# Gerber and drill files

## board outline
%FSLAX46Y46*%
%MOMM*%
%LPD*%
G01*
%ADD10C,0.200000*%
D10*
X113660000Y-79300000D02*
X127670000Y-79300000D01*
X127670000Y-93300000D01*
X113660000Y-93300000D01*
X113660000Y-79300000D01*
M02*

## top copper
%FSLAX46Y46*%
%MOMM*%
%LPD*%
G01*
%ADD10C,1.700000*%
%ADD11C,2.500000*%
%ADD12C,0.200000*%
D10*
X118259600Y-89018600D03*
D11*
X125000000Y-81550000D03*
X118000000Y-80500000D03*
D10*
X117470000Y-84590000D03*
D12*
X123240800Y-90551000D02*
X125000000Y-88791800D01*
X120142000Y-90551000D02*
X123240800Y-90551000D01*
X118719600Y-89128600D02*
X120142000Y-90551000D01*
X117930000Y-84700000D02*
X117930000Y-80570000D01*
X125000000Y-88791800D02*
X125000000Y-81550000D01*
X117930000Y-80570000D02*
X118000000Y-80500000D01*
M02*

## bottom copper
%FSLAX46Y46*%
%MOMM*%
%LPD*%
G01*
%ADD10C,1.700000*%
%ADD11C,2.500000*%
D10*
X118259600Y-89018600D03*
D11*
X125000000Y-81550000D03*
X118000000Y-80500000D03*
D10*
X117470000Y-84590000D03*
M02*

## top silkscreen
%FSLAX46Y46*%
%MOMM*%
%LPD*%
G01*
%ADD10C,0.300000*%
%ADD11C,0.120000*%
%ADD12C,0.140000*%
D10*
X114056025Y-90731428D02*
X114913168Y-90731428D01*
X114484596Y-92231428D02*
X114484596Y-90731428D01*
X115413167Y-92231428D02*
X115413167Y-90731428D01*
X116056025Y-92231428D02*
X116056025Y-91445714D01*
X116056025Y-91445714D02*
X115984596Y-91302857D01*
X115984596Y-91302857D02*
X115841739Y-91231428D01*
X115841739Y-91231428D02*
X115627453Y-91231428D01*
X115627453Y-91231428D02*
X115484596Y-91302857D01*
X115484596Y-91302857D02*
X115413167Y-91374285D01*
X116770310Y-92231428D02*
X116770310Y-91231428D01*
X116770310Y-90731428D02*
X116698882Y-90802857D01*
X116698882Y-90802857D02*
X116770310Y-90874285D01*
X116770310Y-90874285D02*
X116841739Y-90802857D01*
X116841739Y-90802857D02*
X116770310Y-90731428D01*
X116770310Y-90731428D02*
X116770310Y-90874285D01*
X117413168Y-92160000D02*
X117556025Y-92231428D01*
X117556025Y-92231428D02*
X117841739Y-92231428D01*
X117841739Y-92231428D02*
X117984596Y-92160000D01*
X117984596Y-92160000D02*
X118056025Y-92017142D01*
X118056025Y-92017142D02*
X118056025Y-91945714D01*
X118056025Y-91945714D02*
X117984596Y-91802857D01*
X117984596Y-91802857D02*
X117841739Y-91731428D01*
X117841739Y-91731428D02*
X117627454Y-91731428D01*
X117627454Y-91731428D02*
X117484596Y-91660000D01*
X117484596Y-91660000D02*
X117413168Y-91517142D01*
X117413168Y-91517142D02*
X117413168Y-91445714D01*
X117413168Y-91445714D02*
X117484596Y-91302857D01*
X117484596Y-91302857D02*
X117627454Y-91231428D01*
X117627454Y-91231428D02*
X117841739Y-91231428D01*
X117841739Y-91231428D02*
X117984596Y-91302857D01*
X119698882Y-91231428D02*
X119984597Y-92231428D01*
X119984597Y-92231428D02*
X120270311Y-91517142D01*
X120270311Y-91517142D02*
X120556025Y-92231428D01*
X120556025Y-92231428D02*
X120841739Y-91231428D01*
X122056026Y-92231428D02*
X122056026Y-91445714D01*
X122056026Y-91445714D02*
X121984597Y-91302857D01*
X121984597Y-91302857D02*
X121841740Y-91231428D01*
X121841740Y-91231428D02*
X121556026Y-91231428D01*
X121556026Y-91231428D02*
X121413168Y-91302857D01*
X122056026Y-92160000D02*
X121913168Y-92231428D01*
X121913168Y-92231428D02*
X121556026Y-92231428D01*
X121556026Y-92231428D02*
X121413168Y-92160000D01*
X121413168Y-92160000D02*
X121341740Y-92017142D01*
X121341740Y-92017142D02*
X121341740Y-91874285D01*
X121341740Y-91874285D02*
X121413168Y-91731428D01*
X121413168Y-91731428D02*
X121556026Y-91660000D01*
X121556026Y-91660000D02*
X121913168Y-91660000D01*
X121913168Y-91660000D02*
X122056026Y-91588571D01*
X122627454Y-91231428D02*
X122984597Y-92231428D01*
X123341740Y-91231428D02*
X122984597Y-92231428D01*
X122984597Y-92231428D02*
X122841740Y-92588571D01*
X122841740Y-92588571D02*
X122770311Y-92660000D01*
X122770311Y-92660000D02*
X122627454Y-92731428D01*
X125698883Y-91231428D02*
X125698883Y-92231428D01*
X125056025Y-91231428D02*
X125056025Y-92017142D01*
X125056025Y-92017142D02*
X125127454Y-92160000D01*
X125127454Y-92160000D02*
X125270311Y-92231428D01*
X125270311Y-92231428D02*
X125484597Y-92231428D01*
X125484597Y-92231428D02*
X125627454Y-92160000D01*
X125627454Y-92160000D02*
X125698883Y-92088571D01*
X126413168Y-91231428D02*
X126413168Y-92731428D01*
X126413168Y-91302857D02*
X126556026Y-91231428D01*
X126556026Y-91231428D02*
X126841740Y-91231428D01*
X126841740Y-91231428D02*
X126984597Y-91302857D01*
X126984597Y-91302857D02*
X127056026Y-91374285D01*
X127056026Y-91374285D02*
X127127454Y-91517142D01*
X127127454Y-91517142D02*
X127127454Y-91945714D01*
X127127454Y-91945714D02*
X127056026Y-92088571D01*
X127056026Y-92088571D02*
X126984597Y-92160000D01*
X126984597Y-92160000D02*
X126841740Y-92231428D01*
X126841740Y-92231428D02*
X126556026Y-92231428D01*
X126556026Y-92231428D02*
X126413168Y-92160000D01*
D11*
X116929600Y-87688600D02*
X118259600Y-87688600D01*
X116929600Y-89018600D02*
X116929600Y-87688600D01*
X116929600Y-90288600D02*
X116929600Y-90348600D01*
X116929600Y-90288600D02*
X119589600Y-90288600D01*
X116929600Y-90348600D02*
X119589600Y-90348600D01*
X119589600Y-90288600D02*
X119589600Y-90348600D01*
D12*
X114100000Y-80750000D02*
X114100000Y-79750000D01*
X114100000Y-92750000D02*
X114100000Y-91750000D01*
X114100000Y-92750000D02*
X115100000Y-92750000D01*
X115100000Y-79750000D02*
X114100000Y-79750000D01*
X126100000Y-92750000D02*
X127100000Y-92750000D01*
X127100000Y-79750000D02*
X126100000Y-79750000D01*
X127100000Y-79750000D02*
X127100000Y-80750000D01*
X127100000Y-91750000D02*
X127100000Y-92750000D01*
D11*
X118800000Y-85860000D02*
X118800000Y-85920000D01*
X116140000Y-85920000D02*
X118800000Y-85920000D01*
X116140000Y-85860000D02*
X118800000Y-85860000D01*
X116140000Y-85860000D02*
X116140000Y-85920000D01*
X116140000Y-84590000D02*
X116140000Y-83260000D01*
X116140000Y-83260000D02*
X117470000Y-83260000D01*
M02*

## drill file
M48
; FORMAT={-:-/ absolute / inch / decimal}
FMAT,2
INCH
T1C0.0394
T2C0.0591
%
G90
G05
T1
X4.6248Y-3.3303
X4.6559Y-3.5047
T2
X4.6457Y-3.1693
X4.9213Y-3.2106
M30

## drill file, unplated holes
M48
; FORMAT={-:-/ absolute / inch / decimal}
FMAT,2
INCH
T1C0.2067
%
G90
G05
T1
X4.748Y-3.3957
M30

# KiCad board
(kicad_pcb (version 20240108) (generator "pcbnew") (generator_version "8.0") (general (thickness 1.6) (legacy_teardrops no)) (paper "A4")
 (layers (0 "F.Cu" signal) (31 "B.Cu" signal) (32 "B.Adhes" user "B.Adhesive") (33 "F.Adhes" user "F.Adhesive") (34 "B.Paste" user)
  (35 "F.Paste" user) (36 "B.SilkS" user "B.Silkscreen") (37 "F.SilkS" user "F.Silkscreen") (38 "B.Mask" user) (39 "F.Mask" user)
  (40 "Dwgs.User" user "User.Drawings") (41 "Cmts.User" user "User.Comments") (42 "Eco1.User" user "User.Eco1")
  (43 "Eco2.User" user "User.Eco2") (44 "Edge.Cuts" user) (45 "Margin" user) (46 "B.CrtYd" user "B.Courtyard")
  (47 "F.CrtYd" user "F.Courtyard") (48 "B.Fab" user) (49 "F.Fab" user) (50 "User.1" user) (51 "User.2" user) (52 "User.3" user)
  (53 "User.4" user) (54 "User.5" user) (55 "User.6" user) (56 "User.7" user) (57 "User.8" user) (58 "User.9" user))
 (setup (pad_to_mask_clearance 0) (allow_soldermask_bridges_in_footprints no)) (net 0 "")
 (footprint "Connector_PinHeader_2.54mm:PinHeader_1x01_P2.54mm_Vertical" (layer "F.Cu") (at 118.2596 89.0186)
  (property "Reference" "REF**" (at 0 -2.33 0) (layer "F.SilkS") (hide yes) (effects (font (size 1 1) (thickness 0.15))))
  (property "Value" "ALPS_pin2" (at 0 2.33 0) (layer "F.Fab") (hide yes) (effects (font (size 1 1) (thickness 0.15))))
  (fp_line (start -1.33 -1.33) (end 0 -1.33) (stroke (width 0.12) (type solid)) (layer "F.SilkS"))
  (fp_line (start -1.33 0) (end -1.33 -1.33) (stroke (width 0.12) (type solid)) (layer "F.SilkS"))
  (fp_line (start -1.33 1.27) (end -1.33 1.33) (stroke (width 0.12) (type solid)) (layer "F.SilkS"))
  (fp_line (start -1.33 1.27) (end 1.33 1.27) (stroke (width 0.12) (type solid)) (layer "F.SilkS"))
  (fp_line (start -1.33 1.33) (end 1.33 1.33) (stroke (width 0.12) (type solid)) (layer "F.SilkS"))
  (fp_line (start 1.33 1.27) (end 1.33 1.33) (stroke (width 0.12) (type solid)) (layer "F.SilkS"))
  (pad "2" thru_hole circle (at 0 0) (size 1.7 1.7) (drill 1) (layers "*.Cu" "*.Mask") (remove_unused_layers no)))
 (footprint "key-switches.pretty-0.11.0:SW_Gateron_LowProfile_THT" (layer "F.Cu") (at 120.6 86.25 180)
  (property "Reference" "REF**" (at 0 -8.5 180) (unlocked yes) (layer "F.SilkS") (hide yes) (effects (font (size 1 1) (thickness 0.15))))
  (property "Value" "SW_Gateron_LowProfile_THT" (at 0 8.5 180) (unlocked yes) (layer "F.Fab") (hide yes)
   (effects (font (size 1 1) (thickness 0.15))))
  (fp_line (start 6.5 5.5) (end 6.5 6.5) (stroke (width 0.14) (type solid)) (layer "F.SilkS"))
  (fp_line (start 6.5 -6.5) (end 6.5 -5.5) (stroke (width 0.14) (type solid)) (layer "F.SilkS"))
  (fp_line (start 6.5 -6.5) (end 5.5 -6.5) (stroke (width 0.14) (type solid)) (layer "F.SilkS"))
  (fp_line (start 5.5 6.5) (end 6.5 6.5) (stroke (width 0.14) (type solid)) (layer "F.SilkS"))
  (fp_line (start -5.5 -6.5) (end -6.5 -6.5) (stroke (width 0.14) (type solid)) (layer "F.SilkS"))
  (fp_line (start -6.5 6.5) (end -5.5 6.5) (stroke (width 0.14) (type solid)) (layer "F.SilkS"))
  (fp_line (start -6.5 6.5) (end -6.5 5.5) (stroke (width 0.14) (type solid)) (layer "F.SilkS"))
  (fp_line (start -6.5 -5.5) (end -6.5 -6.5) (stroke (width 0.14) (type solid)) (layer "F.SilkS"))
  (pad "" np_thru_hole circle (at 0 0) (size 5.25 5.25) (drill 5.25) (layers "*.Mask"))
  (pad "1" thru_hole circle (at -4.4 4.7) (size 2.5 2.5) (drill 1.5) (layers "*.Cu" "B.Mask") (remove_unused_layers no))
  (pad "2" thru_hole circle (at 2.6 5.75) (size 2.5 2.5) (drill 1.5) (layers "*.Cu" "B.Mask") (remove_unused_layers no)))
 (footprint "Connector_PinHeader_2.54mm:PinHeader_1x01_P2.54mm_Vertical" (layer "F.Cu") (at 117.47 84.59)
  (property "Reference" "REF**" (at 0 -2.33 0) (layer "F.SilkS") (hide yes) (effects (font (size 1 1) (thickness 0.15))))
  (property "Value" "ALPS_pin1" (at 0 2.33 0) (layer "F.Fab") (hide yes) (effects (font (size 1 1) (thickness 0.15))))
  (fp_line (start -1.33 -1.33) (end 0 -1.33) (stroke (width 0.12) (type solid)) (layer "F.SilkS"))
  (fp_line (start -1.33 0) (end -1.33 -1.33) (stroke (width 0.12) (type solid)) (layer "F.SilkS"))
  (fp_line (start -1.33 1.27) (end -1.33 1.33) (stroke (width 0.12) (type solid)) (layer "F.SilkS"))
  (fp_line (start -1.33 1.27) (end 1.33 1.27) (stroke (width 0.12) (type solid)) (layer "F.SilkS"))
  (fp_line (start -1.33 1.33) (end 1.33 1.33) (stroke (width 0.12) (type solid)) (layer "F.SilkS"))
  (fp_line (start 1.33 1.27) (end 1.33 1.33) (stroke (width 0.12) (type solid)) (layer "F.SilkS"))
  (pad "1" thru_hole circle (at 0 0) (size 1.7 1.7) (drill 1) (layers "*.Cu" "*.Mask") (remove_unused_layers no)))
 (gr_rect (start 113.66 79.3) (end 127.67 93.3) (stroke (width 0.2) (type default)) (fill none) (layer "Edge.Cuts"))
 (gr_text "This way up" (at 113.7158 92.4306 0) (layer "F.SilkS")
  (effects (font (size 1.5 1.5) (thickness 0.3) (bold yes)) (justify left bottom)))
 (segment (start 123.2408 90.551) (end 125 88.7918) (width 0.2) (layer "F.Cu") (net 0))
 (segment (start 120.142 90.551) (end 123.2408 90.551) (width 0.2) (layer "F.Cu") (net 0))
 (segment (start 118.7196 89.1286) (end 120.142 90.551) (width 0.2) (layer "F.Cu") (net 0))
 (segment (start 117.93 84.7) (end 117.93 80.57) (width 0.2) (layer "F.Cu") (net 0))
 (segment (start 125 88.7918) (end 125 81.55) (width 0.2) (layer "F.Cu") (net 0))
 (segment (start 117.93 80.57) (end 118 80.5) (width 0.2) (layer "F.Cu") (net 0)))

